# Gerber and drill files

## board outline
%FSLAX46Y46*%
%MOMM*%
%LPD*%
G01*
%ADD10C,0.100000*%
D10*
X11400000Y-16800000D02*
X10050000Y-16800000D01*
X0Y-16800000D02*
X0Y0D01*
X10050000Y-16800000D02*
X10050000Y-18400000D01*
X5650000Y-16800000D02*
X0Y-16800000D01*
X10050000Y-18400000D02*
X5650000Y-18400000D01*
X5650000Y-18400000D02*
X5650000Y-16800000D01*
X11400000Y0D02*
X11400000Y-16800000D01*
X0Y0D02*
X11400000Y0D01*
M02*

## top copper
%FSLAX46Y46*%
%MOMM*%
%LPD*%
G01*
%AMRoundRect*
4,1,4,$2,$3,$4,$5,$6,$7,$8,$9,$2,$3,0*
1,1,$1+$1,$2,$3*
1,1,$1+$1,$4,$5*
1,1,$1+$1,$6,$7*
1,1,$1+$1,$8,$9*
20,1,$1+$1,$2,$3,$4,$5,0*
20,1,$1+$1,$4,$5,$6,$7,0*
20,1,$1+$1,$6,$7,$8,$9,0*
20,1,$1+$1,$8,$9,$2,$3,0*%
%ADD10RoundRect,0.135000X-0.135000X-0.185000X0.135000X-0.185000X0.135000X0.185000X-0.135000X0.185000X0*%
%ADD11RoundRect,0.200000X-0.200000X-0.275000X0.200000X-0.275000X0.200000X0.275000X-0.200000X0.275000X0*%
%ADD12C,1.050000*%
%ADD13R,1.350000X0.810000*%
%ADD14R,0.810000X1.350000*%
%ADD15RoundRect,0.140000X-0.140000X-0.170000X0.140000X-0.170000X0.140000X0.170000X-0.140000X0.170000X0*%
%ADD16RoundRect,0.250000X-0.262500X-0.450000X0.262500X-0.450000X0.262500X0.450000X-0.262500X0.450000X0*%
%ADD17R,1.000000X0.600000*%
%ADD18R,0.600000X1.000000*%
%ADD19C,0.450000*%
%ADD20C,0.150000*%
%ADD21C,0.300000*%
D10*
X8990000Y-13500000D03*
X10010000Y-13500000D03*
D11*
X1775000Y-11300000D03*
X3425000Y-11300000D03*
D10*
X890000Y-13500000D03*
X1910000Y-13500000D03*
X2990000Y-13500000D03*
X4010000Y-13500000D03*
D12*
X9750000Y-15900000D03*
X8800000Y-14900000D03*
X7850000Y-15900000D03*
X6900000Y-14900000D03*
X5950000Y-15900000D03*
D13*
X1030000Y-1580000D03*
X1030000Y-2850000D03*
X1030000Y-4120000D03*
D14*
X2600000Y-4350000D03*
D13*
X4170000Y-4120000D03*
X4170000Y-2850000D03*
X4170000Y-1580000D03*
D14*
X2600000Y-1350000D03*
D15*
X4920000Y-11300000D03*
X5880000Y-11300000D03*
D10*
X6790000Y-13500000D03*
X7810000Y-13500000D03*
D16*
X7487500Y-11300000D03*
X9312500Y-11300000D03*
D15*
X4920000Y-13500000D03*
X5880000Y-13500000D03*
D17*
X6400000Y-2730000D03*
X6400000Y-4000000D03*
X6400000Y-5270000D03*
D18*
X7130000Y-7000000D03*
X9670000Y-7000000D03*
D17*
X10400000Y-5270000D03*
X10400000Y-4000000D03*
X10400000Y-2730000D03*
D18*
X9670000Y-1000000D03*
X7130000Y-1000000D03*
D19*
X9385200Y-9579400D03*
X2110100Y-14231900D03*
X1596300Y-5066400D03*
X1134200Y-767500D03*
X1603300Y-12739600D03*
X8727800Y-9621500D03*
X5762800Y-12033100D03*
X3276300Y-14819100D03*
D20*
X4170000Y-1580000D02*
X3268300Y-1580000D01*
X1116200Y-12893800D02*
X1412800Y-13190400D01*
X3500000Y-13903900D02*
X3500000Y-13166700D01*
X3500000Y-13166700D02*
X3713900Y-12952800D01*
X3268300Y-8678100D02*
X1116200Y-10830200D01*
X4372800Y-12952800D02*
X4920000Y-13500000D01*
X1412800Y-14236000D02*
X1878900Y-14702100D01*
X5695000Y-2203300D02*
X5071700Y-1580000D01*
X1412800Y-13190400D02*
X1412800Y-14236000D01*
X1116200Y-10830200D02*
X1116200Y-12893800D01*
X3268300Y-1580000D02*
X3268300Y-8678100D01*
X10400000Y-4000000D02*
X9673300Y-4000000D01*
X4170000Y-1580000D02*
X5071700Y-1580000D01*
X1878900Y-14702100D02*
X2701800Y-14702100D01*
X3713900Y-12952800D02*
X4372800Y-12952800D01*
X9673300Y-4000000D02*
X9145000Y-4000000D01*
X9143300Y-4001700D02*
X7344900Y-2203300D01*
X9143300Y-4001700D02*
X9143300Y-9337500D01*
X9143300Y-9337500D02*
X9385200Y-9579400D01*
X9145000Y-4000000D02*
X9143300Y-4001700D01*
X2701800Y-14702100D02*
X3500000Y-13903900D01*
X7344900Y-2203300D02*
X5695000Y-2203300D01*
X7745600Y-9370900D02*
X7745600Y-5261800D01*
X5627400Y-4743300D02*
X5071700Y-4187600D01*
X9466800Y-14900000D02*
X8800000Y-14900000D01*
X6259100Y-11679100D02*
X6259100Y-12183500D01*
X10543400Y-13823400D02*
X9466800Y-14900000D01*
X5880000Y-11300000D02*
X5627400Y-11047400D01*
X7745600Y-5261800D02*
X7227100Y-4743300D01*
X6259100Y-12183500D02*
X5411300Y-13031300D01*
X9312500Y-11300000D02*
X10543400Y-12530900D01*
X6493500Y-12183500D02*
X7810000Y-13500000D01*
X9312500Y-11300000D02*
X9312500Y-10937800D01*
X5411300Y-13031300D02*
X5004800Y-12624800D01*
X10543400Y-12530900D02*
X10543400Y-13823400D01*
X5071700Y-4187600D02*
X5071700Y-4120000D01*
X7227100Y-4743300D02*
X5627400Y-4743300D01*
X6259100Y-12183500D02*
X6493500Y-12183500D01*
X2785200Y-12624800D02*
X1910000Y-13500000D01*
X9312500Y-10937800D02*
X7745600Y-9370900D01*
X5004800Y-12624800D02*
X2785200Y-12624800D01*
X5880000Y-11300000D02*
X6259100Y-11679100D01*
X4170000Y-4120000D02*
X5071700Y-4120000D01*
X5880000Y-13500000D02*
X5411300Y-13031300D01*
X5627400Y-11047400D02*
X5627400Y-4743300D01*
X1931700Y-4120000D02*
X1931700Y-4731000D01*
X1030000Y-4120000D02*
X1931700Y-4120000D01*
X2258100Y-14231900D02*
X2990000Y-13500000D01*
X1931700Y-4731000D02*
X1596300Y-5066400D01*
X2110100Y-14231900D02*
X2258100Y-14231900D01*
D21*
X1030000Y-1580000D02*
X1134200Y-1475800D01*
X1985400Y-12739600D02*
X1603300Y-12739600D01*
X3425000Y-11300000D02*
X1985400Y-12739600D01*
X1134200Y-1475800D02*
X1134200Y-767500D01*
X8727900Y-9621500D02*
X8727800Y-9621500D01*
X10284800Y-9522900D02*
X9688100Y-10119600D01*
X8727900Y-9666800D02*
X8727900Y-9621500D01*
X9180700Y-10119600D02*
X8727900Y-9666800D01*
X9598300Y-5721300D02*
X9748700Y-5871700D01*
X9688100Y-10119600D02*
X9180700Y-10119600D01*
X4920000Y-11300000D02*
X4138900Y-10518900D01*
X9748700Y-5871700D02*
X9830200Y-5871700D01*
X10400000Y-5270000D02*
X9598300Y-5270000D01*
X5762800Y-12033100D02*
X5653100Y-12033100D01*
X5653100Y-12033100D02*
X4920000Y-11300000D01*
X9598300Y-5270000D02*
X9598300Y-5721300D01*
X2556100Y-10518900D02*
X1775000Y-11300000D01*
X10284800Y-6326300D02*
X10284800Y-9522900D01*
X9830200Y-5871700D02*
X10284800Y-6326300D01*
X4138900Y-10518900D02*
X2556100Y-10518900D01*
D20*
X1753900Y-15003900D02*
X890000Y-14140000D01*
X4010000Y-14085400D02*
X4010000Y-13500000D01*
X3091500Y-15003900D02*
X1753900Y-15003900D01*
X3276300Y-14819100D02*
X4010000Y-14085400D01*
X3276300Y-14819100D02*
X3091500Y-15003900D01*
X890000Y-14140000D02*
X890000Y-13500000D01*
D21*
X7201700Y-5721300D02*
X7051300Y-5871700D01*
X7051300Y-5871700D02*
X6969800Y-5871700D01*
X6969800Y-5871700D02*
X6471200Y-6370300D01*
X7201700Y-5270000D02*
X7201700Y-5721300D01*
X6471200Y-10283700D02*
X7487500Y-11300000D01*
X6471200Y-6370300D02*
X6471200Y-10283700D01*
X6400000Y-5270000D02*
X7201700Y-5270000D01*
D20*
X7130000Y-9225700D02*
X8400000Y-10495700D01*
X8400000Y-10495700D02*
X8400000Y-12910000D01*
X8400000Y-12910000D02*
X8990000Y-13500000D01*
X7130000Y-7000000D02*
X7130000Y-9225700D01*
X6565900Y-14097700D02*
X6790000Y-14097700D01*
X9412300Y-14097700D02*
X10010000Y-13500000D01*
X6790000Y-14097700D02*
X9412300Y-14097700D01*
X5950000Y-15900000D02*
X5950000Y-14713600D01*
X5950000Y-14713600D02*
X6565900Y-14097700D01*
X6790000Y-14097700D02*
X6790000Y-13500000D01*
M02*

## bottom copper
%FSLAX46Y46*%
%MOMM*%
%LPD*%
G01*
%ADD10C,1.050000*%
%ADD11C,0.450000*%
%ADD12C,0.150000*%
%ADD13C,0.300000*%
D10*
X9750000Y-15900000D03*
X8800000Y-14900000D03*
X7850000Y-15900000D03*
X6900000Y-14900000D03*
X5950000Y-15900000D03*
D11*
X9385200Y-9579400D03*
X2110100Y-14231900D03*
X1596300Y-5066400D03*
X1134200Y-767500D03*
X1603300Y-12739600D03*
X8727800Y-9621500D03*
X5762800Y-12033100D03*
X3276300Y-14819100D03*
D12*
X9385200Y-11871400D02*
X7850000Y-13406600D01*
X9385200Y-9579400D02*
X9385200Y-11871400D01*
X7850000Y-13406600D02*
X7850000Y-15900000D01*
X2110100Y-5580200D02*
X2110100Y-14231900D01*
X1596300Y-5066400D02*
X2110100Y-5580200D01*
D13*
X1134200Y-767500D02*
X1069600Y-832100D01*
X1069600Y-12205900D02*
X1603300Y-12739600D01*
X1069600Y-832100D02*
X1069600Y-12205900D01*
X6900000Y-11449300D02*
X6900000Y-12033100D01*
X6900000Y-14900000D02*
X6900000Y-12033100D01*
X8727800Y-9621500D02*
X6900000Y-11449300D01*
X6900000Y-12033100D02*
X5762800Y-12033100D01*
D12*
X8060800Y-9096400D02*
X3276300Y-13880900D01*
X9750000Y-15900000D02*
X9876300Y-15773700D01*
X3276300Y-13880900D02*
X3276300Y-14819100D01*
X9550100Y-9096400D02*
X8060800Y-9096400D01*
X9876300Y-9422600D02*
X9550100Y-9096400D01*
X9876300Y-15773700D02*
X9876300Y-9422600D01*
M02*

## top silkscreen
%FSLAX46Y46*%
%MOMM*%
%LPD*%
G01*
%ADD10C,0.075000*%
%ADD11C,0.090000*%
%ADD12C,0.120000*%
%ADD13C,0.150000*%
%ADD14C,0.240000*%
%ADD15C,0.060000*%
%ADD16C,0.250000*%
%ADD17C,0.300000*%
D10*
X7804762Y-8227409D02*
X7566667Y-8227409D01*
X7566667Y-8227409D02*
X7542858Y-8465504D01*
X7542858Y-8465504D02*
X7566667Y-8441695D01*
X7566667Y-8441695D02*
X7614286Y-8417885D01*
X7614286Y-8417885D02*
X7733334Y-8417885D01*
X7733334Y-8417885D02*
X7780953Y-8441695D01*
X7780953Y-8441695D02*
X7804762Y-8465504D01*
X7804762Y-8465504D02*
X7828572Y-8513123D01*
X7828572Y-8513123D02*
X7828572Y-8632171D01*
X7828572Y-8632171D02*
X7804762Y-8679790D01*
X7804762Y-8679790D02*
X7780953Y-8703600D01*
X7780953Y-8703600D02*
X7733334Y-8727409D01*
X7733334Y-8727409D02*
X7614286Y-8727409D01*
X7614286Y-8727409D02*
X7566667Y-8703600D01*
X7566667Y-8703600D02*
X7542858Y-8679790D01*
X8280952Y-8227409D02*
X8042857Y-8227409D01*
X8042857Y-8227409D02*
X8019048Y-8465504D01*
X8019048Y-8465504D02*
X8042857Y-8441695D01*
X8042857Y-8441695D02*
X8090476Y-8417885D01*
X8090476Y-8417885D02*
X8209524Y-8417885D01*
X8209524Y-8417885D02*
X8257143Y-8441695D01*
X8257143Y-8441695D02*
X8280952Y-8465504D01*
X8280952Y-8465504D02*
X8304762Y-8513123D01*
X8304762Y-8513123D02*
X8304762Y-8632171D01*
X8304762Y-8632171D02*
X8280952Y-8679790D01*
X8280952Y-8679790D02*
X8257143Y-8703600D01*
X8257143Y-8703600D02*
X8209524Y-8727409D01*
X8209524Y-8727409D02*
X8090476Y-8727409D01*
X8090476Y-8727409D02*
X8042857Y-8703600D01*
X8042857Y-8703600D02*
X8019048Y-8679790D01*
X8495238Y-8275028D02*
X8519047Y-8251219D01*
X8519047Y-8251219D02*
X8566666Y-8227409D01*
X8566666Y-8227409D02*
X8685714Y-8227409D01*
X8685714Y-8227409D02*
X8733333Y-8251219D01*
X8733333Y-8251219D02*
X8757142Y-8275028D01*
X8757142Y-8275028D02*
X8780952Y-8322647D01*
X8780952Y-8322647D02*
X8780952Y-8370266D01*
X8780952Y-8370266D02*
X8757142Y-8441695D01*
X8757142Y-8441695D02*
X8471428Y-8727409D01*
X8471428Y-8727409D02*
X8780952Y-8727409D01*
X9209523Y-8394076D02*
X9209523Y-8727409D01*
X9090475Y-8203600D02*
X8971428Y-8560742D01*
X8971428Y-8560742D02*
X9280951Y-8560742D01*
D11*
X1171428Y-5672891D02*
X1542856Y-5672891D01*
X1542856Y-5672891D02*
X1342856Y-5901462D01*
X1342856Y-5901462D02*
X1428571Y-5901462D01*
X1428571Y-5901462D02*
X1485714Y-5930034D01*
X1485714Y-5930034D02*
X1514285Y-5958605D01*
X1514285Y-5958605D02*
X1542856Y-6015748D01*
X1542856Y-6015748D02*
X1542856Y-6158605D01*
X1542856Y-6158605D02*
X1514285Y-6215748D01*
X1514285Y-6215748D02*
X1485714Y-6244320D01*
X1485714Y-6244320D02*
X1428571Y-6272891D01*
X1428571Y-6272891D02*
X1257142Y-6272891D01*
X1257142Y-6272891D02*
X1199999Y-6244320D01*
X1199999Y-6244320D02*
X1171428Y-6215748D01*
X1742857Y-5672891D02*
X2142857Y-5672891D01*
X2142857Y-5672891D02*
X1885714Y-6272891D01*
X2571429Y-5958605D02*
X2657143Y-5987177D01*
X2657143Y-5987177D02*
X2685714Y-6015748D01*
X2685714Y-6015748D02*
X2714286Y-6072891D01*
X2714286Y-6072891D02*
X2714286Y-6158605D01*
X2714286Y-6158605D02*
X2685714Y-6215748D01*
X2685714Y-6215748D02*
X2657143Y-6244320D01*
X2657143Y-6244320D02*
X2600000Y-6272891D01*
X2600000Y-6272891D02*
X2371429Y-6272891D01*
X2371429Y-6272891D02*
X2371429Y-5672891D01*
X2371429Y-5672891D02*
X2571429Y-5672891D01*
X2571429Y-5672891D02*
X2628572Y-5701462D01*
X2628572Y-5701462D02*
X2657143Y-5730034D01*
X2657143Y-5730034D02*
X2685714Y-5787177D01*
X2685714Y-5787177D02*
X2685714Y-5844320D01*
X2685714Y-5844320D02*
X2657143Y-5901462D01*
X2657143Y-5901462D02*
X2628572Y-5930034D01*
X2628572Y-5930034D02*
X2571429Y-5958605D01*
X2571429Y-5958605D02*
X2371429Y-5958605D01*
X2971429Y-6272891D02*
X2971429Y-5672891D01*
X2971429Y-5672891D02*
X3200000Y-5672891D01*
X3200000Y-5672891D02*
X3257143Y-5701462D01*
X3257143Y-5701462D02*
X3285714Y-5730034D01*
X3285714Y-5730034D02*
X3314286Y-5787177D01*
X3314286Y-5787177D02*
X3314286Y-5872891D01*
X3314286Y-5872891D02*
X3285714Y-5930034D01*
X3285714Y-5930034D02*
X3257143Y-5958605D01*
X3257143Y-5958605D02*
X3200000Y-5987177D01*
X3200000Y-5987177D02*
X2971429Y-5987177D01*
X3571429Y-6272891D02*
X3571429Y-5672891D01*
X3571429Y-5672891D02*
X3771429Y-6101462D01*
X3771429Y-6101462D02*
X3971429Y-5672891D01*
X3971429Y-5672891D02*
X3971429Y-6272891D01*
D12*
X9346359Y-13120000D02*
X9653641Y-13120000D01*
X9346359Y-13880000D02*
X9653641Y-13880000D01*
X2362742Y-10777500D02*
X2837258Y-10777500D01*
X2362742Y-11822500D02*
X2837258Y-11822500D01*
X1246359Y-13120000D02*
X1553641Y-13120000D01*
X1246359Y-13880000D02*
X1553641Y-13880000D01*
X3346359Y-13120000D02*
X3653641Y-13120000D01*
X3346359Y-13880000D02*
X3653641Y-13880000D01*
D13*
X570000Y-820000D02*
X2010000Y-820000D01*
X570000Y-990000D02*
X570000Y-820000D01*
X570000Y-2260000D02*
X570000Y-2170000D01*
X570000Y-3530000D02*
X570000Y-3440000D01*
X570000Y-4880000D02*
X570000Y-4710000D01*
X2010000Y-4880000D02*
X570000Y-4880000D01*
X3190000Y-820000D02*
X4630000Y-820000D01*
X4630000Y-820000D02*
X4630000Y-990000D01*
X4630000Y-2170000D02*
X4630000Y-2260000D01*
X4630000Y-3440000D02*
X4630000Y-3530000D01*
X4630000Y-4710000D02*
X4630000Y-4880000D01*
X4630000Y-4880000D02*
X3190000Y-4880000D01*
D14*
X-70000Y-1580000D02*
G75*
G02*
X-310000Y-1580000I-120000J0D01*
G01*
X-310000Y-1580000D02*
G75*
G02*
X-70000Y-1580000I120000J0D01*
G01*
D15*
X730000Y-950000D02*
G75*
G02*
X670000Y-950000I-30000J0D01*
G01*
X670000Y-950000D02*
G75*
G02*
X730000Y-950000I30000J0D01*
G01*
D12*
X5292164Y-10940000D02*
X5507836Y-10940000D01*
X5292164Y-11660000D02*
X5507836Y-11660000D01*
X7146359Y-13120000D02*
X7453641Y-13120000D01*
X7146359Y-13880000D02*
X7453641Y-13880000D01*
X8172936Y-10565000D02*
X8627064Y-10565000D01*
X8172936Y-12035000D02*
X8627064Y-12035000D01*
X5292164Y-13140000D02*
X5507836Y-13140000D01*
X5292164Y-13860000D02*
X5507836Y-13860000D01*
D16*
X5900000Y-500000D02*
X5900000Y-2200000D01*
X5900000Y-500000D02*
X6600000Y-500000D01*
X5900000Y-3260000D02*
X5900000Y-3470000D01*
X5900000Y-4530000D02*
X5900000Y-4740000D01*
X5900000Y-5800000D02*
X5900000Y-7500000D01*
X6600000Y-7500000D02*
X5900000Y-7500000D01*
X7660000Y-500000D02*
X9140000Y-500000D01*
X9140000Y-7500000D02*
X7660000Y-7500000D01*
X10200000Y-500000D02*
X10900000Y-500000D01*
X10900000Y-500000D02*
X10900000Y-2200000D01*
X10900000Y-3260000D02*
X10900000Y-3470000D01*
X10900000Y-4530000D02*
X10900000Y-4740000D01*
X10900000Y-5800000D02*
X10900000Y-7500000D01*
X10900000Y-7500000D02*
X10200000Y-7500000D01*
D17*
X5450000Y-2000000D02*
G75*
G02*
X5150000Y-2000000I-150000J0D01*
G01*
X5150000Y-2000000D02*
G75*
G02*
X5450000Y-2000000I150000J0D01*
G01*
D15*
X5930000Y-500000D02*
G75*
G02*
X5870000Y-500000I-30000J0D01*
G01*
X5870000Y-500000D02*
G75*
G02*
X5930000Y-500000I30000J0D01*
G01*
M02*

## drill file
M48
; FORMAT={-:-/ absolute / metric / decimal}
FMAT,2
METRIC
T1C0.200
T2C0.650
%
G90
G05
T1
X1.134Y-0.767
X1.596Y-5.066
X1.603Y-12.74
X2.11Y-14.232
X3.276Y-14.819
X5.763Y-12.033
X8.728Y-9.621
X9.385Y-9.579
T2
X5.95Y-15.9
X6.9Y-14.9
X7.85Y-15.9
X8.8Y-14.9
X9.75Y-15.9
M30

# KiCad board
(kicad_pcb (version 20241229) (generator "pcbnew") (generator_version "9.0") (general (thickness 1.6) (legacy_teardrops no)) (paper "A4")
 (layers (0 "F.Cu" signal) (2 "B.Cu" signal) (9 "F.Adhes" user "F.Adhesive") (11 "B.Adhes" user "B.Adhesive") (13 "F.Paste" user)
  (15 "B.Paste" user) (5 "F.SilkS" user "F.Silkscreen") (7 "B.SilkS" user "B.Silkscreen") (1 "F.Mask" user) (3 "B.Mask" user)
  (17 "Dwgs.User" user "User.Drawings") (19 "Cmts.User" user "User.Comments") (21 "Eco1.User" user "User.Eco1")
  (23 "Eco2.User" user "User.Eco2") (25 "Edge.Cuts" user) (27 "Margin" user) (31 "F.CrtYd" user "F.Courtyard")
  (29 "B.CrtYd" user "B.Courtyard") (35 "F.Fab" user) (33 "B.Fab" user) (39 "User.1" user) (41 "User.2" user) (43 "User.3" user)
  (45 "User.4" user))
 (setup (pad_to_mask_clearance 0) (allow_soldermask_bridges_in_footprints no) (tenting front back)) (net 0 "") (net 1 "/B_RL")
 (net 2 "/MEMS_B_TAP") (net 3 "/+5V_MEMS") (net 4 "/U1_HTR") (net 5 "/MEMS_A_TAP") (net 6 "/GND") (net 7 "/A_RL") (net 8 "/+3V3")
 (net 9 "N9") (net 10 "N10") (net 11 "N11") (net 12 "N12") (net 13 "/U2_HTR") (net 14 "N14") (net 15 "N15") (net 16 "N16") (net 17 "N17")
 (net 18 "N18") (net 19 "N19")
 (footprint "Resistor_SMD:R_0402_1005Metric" (layer "F.Cu") (at 9.5 13.5)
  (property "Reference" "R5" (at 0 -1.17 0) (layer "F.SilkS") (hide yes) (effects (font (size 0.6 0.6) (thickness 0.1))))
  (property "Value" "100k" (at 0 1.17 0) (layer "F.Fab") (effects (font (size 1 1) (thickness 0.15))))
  (fp_line (start -0.153641 -0.38) (end 0.153641 -0.38) (stroke (width 0.12) (type solid)) (layer "F.SilkS"))
  (fp_line (start -0.153641 0.38) (end 0.153641 0.38) (stroke (width 0.12) (type solid)) (layer "F.SilkS"))
  (pad "1" smd roundrect (at -0.51 0) (size 0.54 0.64) (layers "F.Cu" "F.Mask" "F.Paste") (roundrect_rratio 0.25) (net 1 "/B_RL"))
  (pad "2" smd roundrect (at 0.51 0) (size 0.54 0.64) (layers "F.Cu" "F.Mask" "F.Paste") (roundrect_rratio 0.25) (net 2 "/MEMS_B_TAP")))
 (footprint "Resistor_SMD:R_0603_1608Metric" (layer "F.Cu") (at 2.6 11.3)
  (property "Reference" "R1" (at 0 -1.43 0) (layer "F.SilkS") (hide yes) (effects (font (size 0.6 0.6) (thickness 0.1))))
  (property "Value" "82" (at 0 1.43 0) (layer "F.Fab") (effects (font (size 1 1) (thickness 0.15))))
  (fp_line (start -0.237258 -0.5225) (end 0.237258 -0.5225) (stroke (width 0.12) (type solid)) (layer "F.SilkS"))
  (fp_line (start -0.237258 0.5225) (end 0.237258 0.5225) (stroke (width 0.12) (type solid)) (layer "F.SilkS"))
  (pad "1" smd roundrect (at -0.825 0) (size 0.8 0.95) (layers "F.Cu" "F.Mask" "F.Paste") (roundrect_rratio 0.25) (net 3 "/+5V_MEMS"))
  (pad "2" smd roundrect (at 0.825 0) (size 0.8 0.95) (layers "F.Cu" "F.Mask" "F.Paste") (roundrect_rratio 0.25) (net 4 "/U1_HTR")))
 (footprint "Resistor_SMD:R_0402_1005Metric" (layer "F.Cu") (at 1.4 13.5)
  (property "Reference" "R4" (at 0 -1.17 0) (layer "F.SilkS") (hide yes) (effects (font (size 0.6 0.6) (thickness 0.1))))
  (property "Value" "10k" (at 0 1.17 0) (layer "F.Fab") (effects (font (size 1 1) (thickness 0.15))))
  (fp_line (start -0.153641 -0.38) (end 0.153641 -0.38) (stroke (width 0.12) (type solid)) (layer "F.SilkS"))
  (fp_line (start -0.153641 0.38) (end 0.153641 0.38) (stroke (width 0.12) (type solid)) (layer "F.SilkS"))
  (pad "1" smd roundrect (at -0.51 0) (size 0.54 0.64) (layers "F.Cu" "F.Mask" "F.Paste") (roundrect_rratio 0.25) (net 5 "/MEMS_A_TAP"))
  (pad "2" smd roundrect (at 0.51 0) (size 0.54 0.64) (layers "F.Cu" "F.Mask" "F.Paste") (roundrect_rratio 0.25) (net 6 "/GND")))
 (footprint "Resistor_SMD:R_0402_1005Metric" (layer "F.Cu") (at 3.5 13.5)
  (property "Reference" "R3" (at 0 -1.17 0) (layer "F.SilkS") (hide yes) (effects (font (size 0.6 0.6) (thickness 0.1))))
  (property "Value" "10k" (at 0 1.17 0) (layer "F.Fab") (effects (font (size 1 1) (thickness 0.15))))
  (fp_line (start -0.153641 -0.38) (end 0.153641 -0.38) (stroke (width 0.12) (type solid)) (layer "F.SilkS"))
  (fp_line (start -0.153641 0.38) (end 0.153641 0.38) (stroke (width 0.12) (type solid)) (layer "F.SilkS"))
  (pad "1" smd roundrect (at -0.51 0) (size 0.54 0.64) (layers "F.Cu" "F.Mask" "F.Paste") (roundrect_rratio 0.25) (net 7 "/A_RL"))
  (pad "2" smd roundrect (at 0.51 0) (size 0.54 0.64) (layers "F.Cu" "F.Mask" "F.Paste") (roundrect_rratio 0.25) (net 5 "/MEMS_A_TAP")))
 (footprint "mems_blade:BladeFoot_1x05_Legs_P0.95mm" (layer "F.Cu") (at 7.85 15.9)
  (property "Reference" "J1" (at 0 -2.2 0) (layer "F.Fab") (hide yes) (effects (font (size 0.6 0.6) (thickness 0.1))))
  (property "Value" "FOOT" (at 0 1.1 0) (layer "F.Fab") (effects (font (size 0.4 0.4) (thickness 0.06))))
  (pad "1" thru_hole circle (at 1.9 0) (size 1.05 1.05) (drill 0.65) (layers "*.Cu" "*.Mask") (remove_unused_layers no)
   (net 5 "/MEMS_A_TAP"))
  (pad "2" thru_hole circle (at 0.95 -1) (size 1.05 1.05) (drill 0.65) (layers "*.Cu" "*.Mask") (remove_unused_layers no) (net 6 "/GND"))
  (pad "3" thru_hole circle (at 0 0) (size 1.05 1.05) (drill 0.65) (layers "*.Cu" "*.Mask") (remove_unused_layers no) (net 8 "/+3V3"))
  (pad "4" thru_hole circle (at -0.95 -1) (size 1.05 1.05) (drill 0.65) (layers "*.Cu" "*.Mask") (remove_unused_layers no)
   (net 3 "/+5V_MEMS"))
  (pad "5" thru_hole circle (at -1.9 0) (size 1.05 1.05) (drill 0.65) (layers "*.Cu" "*.Mask") (remove_unused_layers no)
   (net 2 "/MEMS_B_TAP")))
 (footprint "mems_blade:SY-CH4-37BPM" (layer "F.Cu") (at 2.6 2.85)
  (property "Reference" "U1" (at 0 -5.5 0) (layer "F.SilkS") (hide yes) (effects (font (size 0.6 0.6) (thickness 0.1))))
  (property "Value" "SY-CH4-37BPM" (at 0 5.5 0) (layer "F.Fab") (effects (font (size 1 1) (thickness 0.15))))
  (fp_line (start -2.03 -2.03) (end -0.59 -2.03) (stroke (width 0.15) (type solid)) (layer "F.SilkS"))
  (fp_line (start -2.03 -1.86) (end -2.03 -2.03) (stroke (width 0.15) (type solid)) (layer "F.SilkS"))
  (fp_line (start -2.03 -0.59) (end -2.03 -0.68) (stroke (width 0.15) (type solid)) (layer "F.SilkS"))
  (fp_line (start -2.03 0.68) (end -2.03 0.59) (stroke (width 0.15) (type solid)) (layer "F.SilkS"))
  (fp_line (start -2.03 2.03) (end -2.03 1.86) (stroke (width 0.15) (type solid)) (layer "F.SilkS"))
  (fp_line (start -0.59 2.03) (end -2.03 2.03) (stroke (width 0.15) (type solid)) (layer "F.SilkS"))
  (fp_line (start 0.59 -2.03) (end 2.03 -2.03) (stroke (width 0.15) (type solid)) (layer "F.SilkS"))
  (fp_line (start 2.03 -2.03) (end 2.03 -1.86) (stroke (width 0.15) (type solid)) (layer "F.SilkS"))
  (fp_line (start 2.03 -0.68) (end 2.03 -0.59) (stroke (width 0.15) (type solid)) (layer "F.SilkS"))
  (fp_line (start 2.03 0.59) (end 2.03 0.68) (stroke (width 0.15) (type solid)) (layer "F.SilkS"))
  (fp_line (start 2.03 1.86) (end 2.03 2.03) (stroke (width 0.15) (type solid)) (layer "F.SilkS"))
  (fp_line (start 2.03 2.03) (end 0.59 2.03) (stroke (width 0.15) (type solid)) (layer "F.SilkS"))
  (fp_circle (center -2.79 -1.27) (end -2.67 -1.27) (stroke (width 0.24) (type solid)) (fill no) (layer "F.SilkS"))
  (fp_circle (center -1.9 -1.9) (end -1.87 -1.9) (stroke (width 0.06) (type solid)) (fill no) (layer "F.SilkS"))
  (pad "1" smd rect (at -1.57 -1.27) (size 1.35 0.81) (layers "F.Cu" "F.Mask" "F.Paste") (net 4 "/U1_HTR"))
  (pad "2" smd rect (at -1.57 0) (size 1.35 0.81) (layers "F.Cu" "F.Mask" "F.Paste") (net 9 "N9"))
  (pad "3" smd rect (at -1.57 1.27) (size 1.35 0.81) (layers "F.Cu" "F.Mask" "F.Paste") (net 7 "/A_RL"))
  (pad "4" smd rect (at 0 1.5 270) (size 1.35 0.81) (layers "F.Cu" "F.Mask" "F.Paste") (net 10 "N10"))
  (pad "5" smd rect (at 1.57 1.27 270) (size 0.81 1.35) (layers "F.Cu" "F.Mask" "F.Paste") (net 6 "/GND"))
  (pad "6" smd rect (at 1.57 0 270) (size 0.81 1.35) (layers "F.Cu" "F.Mask" "F.Paste") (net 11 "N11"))
  (pad "7" smd rect (at 1.57 -1.27 270) (size 0.81 1.35) (layers "F.Cu" "F.Mask" "F.Paste") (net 8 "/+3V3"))
  (pad "8" smd rect (at 0 -1.5 270) (size 1.35 0.81) (layers "F.Cu" "F.Mask" "F.Paste") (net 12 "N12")))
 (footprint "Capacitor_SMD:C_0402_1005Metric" (layer "F.Cu") (at 5.4 11.3)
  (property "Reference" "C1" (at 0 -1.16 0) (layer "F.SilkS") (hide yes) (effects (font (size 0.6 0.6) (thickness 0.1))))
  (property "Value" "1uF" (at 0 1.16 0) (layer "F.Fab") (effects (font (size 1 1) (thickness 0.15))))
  (fp_line (start -0.107836 -0.36) (end 0.107836 -0.36) (stroke (width 0.12) (type solid)) (layer "F.SilkS"))
  (fp_line (start -0.107836 0.36) (end 0.107836 0.36) (stroke (width 0.12) (type solid)) (layer "F.SilkS"))
  (pad "1" smd roundrect (at -0.48 0) (size 0.56 0.62) (layers "F.Cu" "F.Mask" "F.Paste") (roundrect_rratio 0.25) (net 3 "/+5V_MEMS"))
  (pad "2" smd roundrect (at 0.48 0) (size 0.56 0.62) (layers "F.Cu" "F.Mask" "F.Paste") (roundrect_rratio 0.25) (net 6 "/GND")))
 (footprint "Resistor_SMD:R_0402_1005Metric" (layer "F.Cu") (at 7.3 13.5)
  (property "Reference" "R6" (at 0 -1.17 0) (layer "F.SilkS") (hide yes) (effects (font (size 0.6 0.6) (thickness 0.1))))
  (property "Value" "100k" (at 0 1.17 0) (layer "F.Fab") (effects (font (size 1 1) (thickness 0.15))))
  (fp_line (start -0.153641 -0.38) (end 0.153641 -0.38) (stroke (width 0.12) (type solid)) (layer "F.SilkS"))
  (fp_line (start -0.153641 0.38) (end 0.153641 0.38) (stroke (width 0.12) (type solid)) (layer "F.SilkS"))
  (pad "1" smd roundrect (at -0.51 0) (size 0.54 0.64) (layers "F.Cu" "F.Mask" "F.Paste") (roundrect_rratio 0.25) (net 2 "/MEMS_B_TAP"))
  (pad "2" smd roundrect (at 0.51 0) (size 0.54 0.64) (layers "F.Cu" "F.Mask" "F.Paste") (roundrect_rratio 0.25) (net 6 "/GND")))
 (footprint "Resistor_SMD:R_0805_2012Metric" (layer "F.Cu") (at 8.4 11.3)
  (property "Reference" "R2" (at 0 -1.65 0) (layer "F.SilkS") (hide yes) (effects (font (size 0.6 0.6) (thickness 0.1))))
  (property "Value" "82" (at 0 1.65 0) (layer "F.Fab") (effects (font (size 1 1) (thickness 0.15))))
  (fp_line (start -0.227064 -0.735) (end 0.227064 -0.735) (stroke (width 0.12) (type solid)) (layer "F.SilkS"))
  (fp_line (start -0.227064 0.735) (end 0.227064 0.735) (stroke (width 0.12) (type solid)) (layer "F.SilkS"))
  (pad "1" smd roundrect (at -0.9125 0) (size 1.025 1.4) (layers "F.Cu" "F.Mask" "F.Paste") (roundrect_rratio 0.243902) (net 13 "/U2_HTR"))
  (pad "2" smd roundrect (at 0.9125 0) (size 1.025 1.4) (layers "F.Cu" "F.Mask" "F.Paste") (roundrect_rratio 0.243902) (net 6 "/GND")))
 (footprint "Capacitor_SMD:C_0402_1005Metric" (layer "F.Cu") (at 5.4 13.5)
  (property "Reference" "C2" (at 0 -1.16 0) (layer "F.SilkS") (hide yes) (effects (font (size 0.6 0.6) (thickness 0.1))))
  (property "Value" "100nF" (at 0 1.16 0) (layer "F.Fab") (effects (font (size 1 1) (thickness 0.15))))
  (fp_line (start -0.107836 -0.36) (end 0.107836 -0.36) (stroke (width 0.12) (type solid)) (layer "F.SilkS"))
  (fp_line (start -0.107836 0.36) (end 0.107836 0.36) (stroke (width 0.12) (type solid)) (layer "F.SilkS"))
  (pad "1" smd roundrect (at -0.48 0) (size 0.56 0.62) (layers "F.Cu" "F.Mask" "F.Paste") (roundrect_rratio 0.25) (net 8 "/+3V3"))
  (pad "2" smd roundrect (at 0.48 0) (size 0.56 0.62) (layers "F.Cu" "F.Mask" "F.Paste") (roundrect_rratio 0.25) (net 6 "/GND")))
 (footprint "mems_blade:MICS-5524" (layer "F.Cu") (at 8.4 4 90)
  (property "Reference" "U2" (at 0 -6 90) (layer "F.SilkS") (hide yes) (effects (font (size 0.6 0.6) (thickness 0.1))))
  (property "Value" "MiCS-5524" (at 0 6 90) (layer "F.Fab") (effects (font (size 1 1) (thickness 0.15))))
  (fp_line (start 3.5 -2.5) (end 1.8 -2.5) (stroke (width 0.25) (type solid)) (layer "F.SilkS"))
  (fp_line (start 3.5 -2.5) (end 3.5 -1.8) (stroke (width 0.25) (type solid)) (layer "F.SilkS"))
  (fp_line (start 0.74 -2.5) (end 0.53 -2.5) (stroke (width 0.25) (type solid)) (layer "F.SilkS"))
  (fp_line (start -0.53 -2.5) (end -0.74 -2.5) (stroke (width 0.25) (type solid)) (layer "F.SilkS"))
  (fp_line (start -1.8 -2.5) (end -3.5 -2.5) (stroke (width 0.25) (type solid)) (layer "F.SilkS"))
  (fp_line (start -3.5 -1.8) (end -3.5 -2.5) (stroke (width 0.25) (type solid)) (layer "F.SilkS"))
  (fp_line (start 3.5 -0.74) (end 3.5 0.74) (stroke (width 0.25) (type solid)) (layer "F.SilkS"))
  (fp_line (start -3.5 0.74) (end -3.5 -0.74) (stroke (width 0.25) (type solid)) (layer "F.SilkS"))
  (fp_line (start 3.5 1.8) (end 3.5 2.5) (stroke (width 0.25) (type solid)) (layer "F.SilkS"))
  (fp_line (start 3.5 2.5) (end 1.8 2.5) (stroke (width 0.25) (type solid)) (layer "F.SilkS"))
  (fp_line (start 0.74 2.5) (end 0.53 2.5) (stroke (width 0.25) (type solid)) (layer "F.SilkS"))
  (fp_line (start -0.53 2.5) (end -0.74 2.5) (stroke (width 0.25) (type solid)) (layer "F.SilkS"))
  (fp_line (start -1.8 2.5) (end -3.5 2.5) (stroke (width 0.25) (type solid)) (layer "F.SilkS"))
  (fp_line (start -3.5 2.5) (end -3.5 1.8) (stroke (width 0.25) (type solid)) (layer "F.SilkS"))
  (fp_circle (center 2 -3.1) (end 2.15 -3.1) (stroke (width 0.3) (type solid)) (fill no) (layer "F.SilkS"))
  (fp_circle (center 3.5 -2.5) (end 3.53 -2.5) (stroke (width 0.06) (type solid)) (fill no) (layer "F.SilkS"))
  (pad "A" smd rect (at 1.27 -2 270) (size 0.6 1) (layers "F.Cu" "F.Mask" "F.Paste") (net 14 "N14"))
  (pad "B" smd rect (at 0 -2 270) (size 0.6 1) (layers "F.Cu" "F.Mask" "F.Paste") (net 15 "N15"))
  (pad "C" smd rect (at -1.27 -2 270) (size 0.6 1) (layers "F.Cu" "F.Mask" "F.Paste") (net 13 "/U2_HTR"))
  (pad "D" smd rect (at -3 -1.27) (size 0.6 1) (layers "F.Cu" "F.Mask" "F.Paste") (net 1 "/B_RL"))
  (pad "E" smd rect (at -3 1.27) (size 0.6 1) (layers "F.Cu" "F.Mask" "F.Paste") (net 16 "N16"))
  (pad "F" smd rect (at -1.27 2 270) (size 0.6 1) (layers "F.Cu" "F.Mask" "F.Paste") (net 3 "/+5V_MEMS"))
  (pad "G" smd rect (at 0 2 270) (size 0.6 1) (layers "F.Cu" "F.Mask" "F.Paste") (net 8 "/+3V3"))
  (pad "H" smd rect (at 1.27 2 270) (size 0.6 1) (layers "F.Cu" "F.Mask" "F.Paste") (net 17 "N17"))
  (pad "J" smd rect (at 3 1.27) (size 0.6 1) (layers "F.Cu" "F.Mask" "F.Paste") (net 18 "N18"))
  (pad "K" smd rect (at 3 -1.27) (size 0.6 1) (layers "F.Cu" "F.Mask" "F.Paste") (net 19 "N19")))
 (gr_line (start 11.4 16.8) (end 10.05 16.8) (stroke (width 0.1) (type default)) (layer "Edge.Cuts"))
 (gr_line (start 0 16.8) (end 0 0) (stroke (width 0.1) (type default)) (layer "Edge.Cuts"))
 (gr_line (start 10.05 16.8) (end 10.05 18.4) (stroke (width 0.1) (type default)) (layer "Edge.Cuts"))
 (gr_line (start 5.65 16.8) (end 0 16.8) (stroke (width 0.1) (type default)) (layer "Edge.Cuts"))
 (gr_line (start 10.05 18.4) (end 5.65 18.4) (stroke (width 0.1) (type default)) (layer "Edge.Cuts"))
 (gr_line (start 5.65 18.4) (end 5.65 16.8) (stroke (width 0.1) (type default)) (layer "Edge.Cuts"))
 (gr_line (start 11.4 0) (end 11.4 16.8) (stroke (width 0.1) (type default)) (layer "Edge.Cuts"))
 (gr_line (start 0 0) (end 11.4 0) (stroke (width 0.1) (type default)) (layer "Edge.Cuts"))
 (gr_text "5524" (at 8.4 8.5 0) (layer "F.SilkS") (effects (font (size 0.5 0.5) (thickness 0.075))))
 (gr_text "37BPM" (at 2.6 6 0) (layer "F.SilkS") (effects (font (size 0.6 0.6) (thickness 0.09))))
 (segment (start 4.17 1.58) (end 3.2683 1.58) (width 0.15) (layer "F.Cu") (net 8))
 (segment (start 1.1162 12.8938) (end 1.4128 13.1904) (width 0.15) (layer "F.Cu") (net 8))
 (segment (start 3.5 13.9039) (end 3.5 13.1667) (width 0.15) (layer "F.Cu") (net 8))
 (segment (start 3.5 13.1667) (end 3.7139 12.9528) (width 0.15) (layer "F.Cu") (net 8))
 (segment (start 3.2683 8.6781) (end 1.1162 10.8302) (width 0.15) (layer "F.Cu") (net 8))
 (segment (start 4.3728 12.9528) (end 4.92 13.5) (width 0.15) (layer "F.Cu") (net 8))
 (segment (start 1.4128 14.236) (end 1.8789 14.7021) (width 0.15) (layer "F.Cu") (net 8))
 (segment (start 5.695 2.2033) (end 5.0717 1.58) (width 0.15) (layer "F.Cu") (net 8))
 (segment (start 1.4128 13.1904) (end 1.4128 14.236) (width 0.15) (layer "F.Cu") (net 8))
 (segment (start 1.1162 10.8302) (end 1.1162 12.8938) (width 0.15) (layer "F.Cu") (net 8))
 (segment (start 3.2683 1.58) (end 3.2683 8.6781) (width 0.15) (layer "F.Cu") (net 8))
 (segment (start 10.4 4) (end 9.6733 4) (width 0.15) (layer "F.Cu") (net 8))
 (segment (start 4.17 1.58) (end 5.0717 1.58) (width 0.15) (layer "F.Cu") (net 8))
 (segment (start 1.8789 14.7021) (end 2.7018 14.7021) (width 0.15) (layer "F.Cu") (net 8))
 (segment (start 3.7139 12.9528) (end 4.3728 12.9528) (width 0.15) (layer "F.Cu") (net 8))
 (segment (start 9.6733 4) (end 9.145 4) (width 0.15) (layer "F.Cu") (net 8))
 (segment (start 9.1433 4.0017) (end 7.3449 2.2033) (width 0.15) (layer "F.Cu") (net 8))
 (segment (start 9.1433 4.0017) (end 9.1433 9.3375) (width 0.15) (layer "F.Cu") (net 8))
 (segment (start 9.1433 9.3375) (end 9.3852 9.5794) (width 0.15) (layer "F.Cu") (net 8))
 (segment (start 9.145 4) (end 9.1433 4.0017) (width 0.15) (layer "F.Cu") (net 8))
 (segment (start 2.7018 14.7021) (end 3.5 13.9039) (width 0.15) (layer "F.Cu") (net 8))
 (segment (start 7.3449 2.2033) (end 5.695 2.2033) (width 0.15) (layer "F.Cu") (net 8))
 (via (at 9.3852 9.5794) (size 0.45) (drill 0.2) (layers "F.Cu" "B.Cu") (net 8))
 (segment (start 9.3852 11.8714) (end 7.85 13.4066) (width 0.15) (layer "B.Cu") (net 8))
 (segment (start 9.3852 9.5794) (end 9.3852 11.8714) (width 0.15) (layer "B.Cu") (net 8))
 (segment (start 7.85 13.4066) (end 7.85 15.9) (width 0.15) (layer "B.Cu") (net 8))
 (segment (start 7.7456 9.3709) (end 7.7456 5.2618) (width 0.15) (layer "F.Cu") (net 6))
 (segment (start 5.6274 4.7433) (end 5.0717 4.1876) (width 0.15) (layer "F.Cu") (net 6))
 (segment (start 9.4668 14.9) (end 8.8 14.9) (width 0.15) (layer "F.Cu") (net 6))
 (segment (start 6.2591 11.6791) (end 6.2591 12.1835) (width 0.15) (layer "F.Cu") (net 6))
 (segment (start 10.5434 13.8234) (end 9.4668 14.9) (width 0.15) (layer "F.Cu") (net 6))
 (segment (start 5.88 11.3) (end 5.6274 11.0474) (width 0.15) (layer "F.Cu") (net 6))
 (segment (start 7.7456 5.2618) (end 7.2271 4.7433) (width 0.15) (layer "F.Cu") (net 6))
 (segment (start 6.2591 12.1835) (end 5.4113 13.0313) (width 0.15) (layer "F.Cu") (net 6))
 (segment (start 9.3125 11.3) (end 10.5434 12.5309) (width 0.15) (layer "F.Cu") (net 6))
 (segment (start 6.4935 12.1835) (end 7.81 13.5) (width 0.15) (layer "F.Cu") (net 6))
 (segment (start 9.3125 11.3) (end 9.3125 10.9378) (width 0.15) (layer "F.Cu") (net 6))
 (segment (start 5.4113 13.0313) (end 5.0048 12.6248) (width 0.15) (layer "F.Cu") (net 6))
 (segment (start 10.5434 12.5309) (end 10.5434 13.8234) (width 0.15) (layer "F.Cu") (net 6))
 (segment (start 5.0717 4.1876) (end 5.0717 4.12) (width 0.15) (layer "F.Cu") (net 6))
 (segment (start 7.2271 4.7433) (end 5.6274 4.7433) (width 0.15) (layer "F.Cu") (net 6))
 (segment (start 6.2591 12.1835) (end 6.4935 12.1835) (width 0.15) (layer "F.Cu") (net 6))
 (segment (start 2.7852 12.6248) (end 1.91 13.5) (width 0.15) (layer "F.Cu") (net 6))
 (segment (start 9.3125 10.9378) (end 7.7456 9.3709) (width 0.15) (layer "F.Cu") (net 6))
 (segment (start 5.0048 12.6248) (end 2.7852 12.6248) (width 0.15) (layer "F.Cu") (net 6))
 (segment (start 5.88 11.3) (end 6.2591 11.6791) (width 0.15) (layer "F.Cu") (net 6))
 (segment (start 4.17 4.12) (end 5.0717 4.12) (width 0.15) (layer "F.Cu") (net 6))
 (segment (start 5.88 13.5) (end 5.4113 13.0313) (width 0.15) (layer "F.Cu") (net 6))
 (segment (start 5.6274 11.0474) (end 5.6274 4.7433) (width 0.15) (layer "F.Cu") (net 6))
 (segment (start 1.9317 4.12) (end 1.9317 4.731) (width 0.15) (layer "F.Cu") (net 7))
 (segment (start 1.03 4.12) (end 1.9317 4.12) (width 0.15) (layer "F.Cu") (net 7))
 (segment (start 2.2581 14.2319) (end 2.99 13.5) (width 0.15) (layer "F.Cu") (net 7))
 (segment (start 1.9317 4.731) (end 1.5963 5.0664) (width 0.15) (layer "F.Cu") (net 7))
 (segment (start 2.1101 14.2319) (end 2.2581 14.2319) (width 0.15) (layer "F.Cu") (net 7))
 (via (at 2.1101 14.2319) (size 0.45) (drill 0.2) (layers "F.Cu" "B.Cu") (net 7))
 (via (at 1.5963 5.0664) (size 0.45) (drill 0.2) (layers "F.Cu" "B.Cu") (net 7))
 (segment (start 2.1101 5.5802) (end 2.1101 14.2319) (width 0.15) (layer "B.Cu") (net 7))
 (segment (start 1.5963 5.0664) (end 2.1101 5.5802) (width 0.15) (layer "B.Cu") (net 7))
 (segment (start 1.03 1.58) (end 1.1342 1.4758) (width 0.3) (layer "F.Cu") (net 4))
 (segment (start 1.9854 12.7396) (end 1.6033 12.7396) (width 0.3) (layer "F.Cu") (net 4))
 (segment (start 3.425 11.3) (end 1.9854 12.7396) (width 0.3) (layer "F.Cu") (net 4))
 (segment (start 1.1342 1.4758) (end 1.1342 0.7675) (width 0.3) (layer "F.Cu") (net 4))
 (via (at 1.1342 0.7675) (size 0.45) (drill 0.2) (layers "F.Cu" "B.Cu") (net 4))
 (via (at 1.6033 12.7396) (size 0.45) (drill 0.2) (layers "F.Cu" "B.Cu") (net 4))
 (segment (start 1.1342 0.7675) (end 1.0696 0.8321) (width 0.3) (layer "B.Cu") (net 4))
 (segment (start 1.0696 12.2059) (end 1.6033 12.7396) (width 0.3) (layer "B.Cu") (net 4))
 (segment (start 1.0696 0.8321) (end 1.0696 12.2059) (width 0.3) (layer "B.Cu") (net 4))
 (segment (start 8.7279 9.6215) (end 8.7278 9.6215) (width 0.3) (layer "F.Cu") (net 3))
 (segment (start 10.2848 9.5229) (end 9.6881 10.1196) (width 0.3) (layer "F.Cu") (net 3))
 (segment (start 8.7279 9.6668) (end 8.7279 9.6215) (width 0.3) (layer "F.Cu") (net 3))
 (segment (start 9.1807 10.1196) (end 8.7279 9.6668) (width 0.3) (layer "F.Cu") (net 3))
 (segment (start 9.5983 5.7213) (end 9.7487 5.8717) (width 0.3) (layer "F.Cu") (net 3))
 (segment (start 9.6881 10.1196) (end 9.1807 10.1196) (width 0.3) (layer "F.Cu") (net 3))
 (segment (start 4.92 11.3) (end 4.1389 10.5189) (width 0.3) (layer "F.Cu") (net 3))
 (segment (start 9.7487 5.8717) (end 9.8302 5.8717) (width 0.3) (layer "F.Cu") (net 3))
 (segment (start 10.4 5.27) (end 9.5983 5.27) (width 0.3) (layer "F.Cu") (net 3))
 (segment (start 5.7628 12.0331) (end 5.6531 12.0331) (width 0.3) (layer "F.Cu") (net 3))
 (segment (start 5.6531 12.0331) (end 4.92 11.3) (width 0.3) (layer "F.Cu") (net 3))
 (segment (start 9.5983 5.27) (end 9.5983 5.7213) (width 0.3) (layer "F.Cu") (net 3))
 (segment (start 2.5561 10.5189) (end 1.775 11.3) (width 0.3) (layer "F.Cu") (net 3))
 (segment (start 10.2848 6.3263) (end 10.2848 9.5229) (width 0.3) (layer "F.Cu") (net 3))
 (segment (start 9.8302 5.8717) (end 10.2848 6.3263) (width 0.3) (layer "F.Cu") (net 3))
 (segment (start 4.1389 10.5189) (end 2.5561 10.5189) (width 0.3) (layer "F.Cu") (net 3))
 (via (at 8.7278 9.6215) (size 0.45) (drill 0.2) (layers "F.Cu" "B.Cu") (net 3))
 (via (at 5.7628 12.0331) (size 0.45) (drill 0.2) (layers "F.Cu" "B.Cu") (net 3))
 (segment (start 6.9 11.4493) (end 6.9 12.0331) (width 0.3) (layer "B.Cu") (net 3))
 (segment (start 6.9 14.9) (end 6.9 12.0331) (width 0.3) (layer "B.Cu") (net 3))
 (segment (start 8.7278 9.6215) (end 6.9 11.4493) (width 0.3) (layer "B.Cu") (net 3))
 (segment (start 6.9 12.0331) (end 5.7628 12.0331) (width 0.3) (layer "B.Cu") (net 3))
 (segment (start 1.7539 15.0039) (end 0.89 14.14) (width 0.15) (layer "F.Cu") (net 5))
 (segment (start 4.01 14.0854) (end 4.01 13.5) (width 0.15) (layer "F.Cu") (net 5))
 (segment (start 3.0915 15.0039) (end 1.7539 15.0039) (width 0.15) (layer "F.Cu") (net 5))
 (segment (start 3.2763 14.8191) (end 4.01 14.0854) (width 0.15) (layer "F.Cu") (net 5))
 (segment (start 3.2763 14.8191) (end 3.0915 15.0039) (width 0.15) (layer "F.Cu") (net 5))
 (segment (start 0.89 14.14) (end 0.89 13.5) (width 0.15) (layer "F.Cu") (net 5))
 (via (at 3.2763 14.8191) (size 0.45) (drill 0.2) (layers "F.Cu" "B.Cu") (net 5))
 (segment (start 8.0608 9.0964) (end 3.2763 13.8809) (width 0.15) (layer "B.Cu") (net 5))
 (segment (start 9.75 15.9) (end 9.8763 15.7737) (width 0.15) (layer "B.Cu") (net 5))
 (segment (start 3.2763 13.8809) (end 3.2763 14.8191) (width 0.15) (layer "B.Cu") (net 5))
 (segment (start 9.5501 9.0964) (end 8.0608 9.0964) (width 0.15) (layer "B.Cu") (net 5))
 (segment (start 9.8763 9.4226) (end 9.5501 9.0964) (width 0.15) (layer "B.Cu") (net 5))
 (segment (start 9.8763 15.7737) (end 9.8763 9.4226) (width 0.15) (layer "B.Cu") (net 5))
 (segment (start 7.2017 5.7213) (end 7.0513 5.8717) (width 0.3) (layer "F.Cu") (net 13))
 (segment (start 7.0513 5.8717) (end 6.9698 5.8717) (width 0.3) (layer "F.Cu") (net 13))
 (segment (start 6.9698 5.8717) (end 6.4712 6.3703) (width 0.3) (layer "F.Cu") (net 13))
 (segment (start 7.2017 5.27) (end 7.2017 5.7213) (width 0.3) (layer "F.Cu") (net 13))
 (segment (start 6.4712 10.2837) (end 7.4875 11.3) (width 0.3) (layer "F.Cu") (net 13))
 (segment (start 6.4712 6.3703) (end 6.4712 10.2837) (width 0.3) (layer "F.Cu") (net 13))
 (segment (start 6.4 5.27) (end 7.2017 5.27) (width 0.3) (layer "F.Cu") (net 13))
 (segment (start 7.13 9.2257) (end 8.4 10.4957) (width 0.15) (layer "F.Cu") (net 1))
 (segment (start 8.4 10.4957) (end 8.4 12.91) (width 0.15) (layer "F.Cu") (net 1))
 (segment (start 8.4 12.91) (end 8.99 13.5) (width 0.15) (layer "F.Cu") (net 1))
 (segment (start 7.13 7) (end 7.13 9.2257) (width 0.15) (layer "F.Cu") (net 1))
 (segment (start 6.5659 14.0977) (end 6.79 14.0977) (width 0.15) (layer "F.Cu") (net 2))
 (segment (start 9.4123 14.0977) (end 10.01 13.5) (width 0.15) (layer "F.Cu") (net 2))
 (segment (start 6.79 14.0977) (end 9.4123 14.0977) (width 0.15) (layer "F.Cu") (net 2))
 (segment (start 5.95 15.9) (end 5.95 14.7136) (width 0.15) (layer "F.Cu") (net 2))
 (segment (start 5.95 14.7136) (end 6.5659 14.0977) (width 0.15) (layer "F.Cu") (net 2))
 (segment (start 6.79 14.0977) (end 6.79 13.5) (width 0.15) (layer "F.Cu") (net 2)))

